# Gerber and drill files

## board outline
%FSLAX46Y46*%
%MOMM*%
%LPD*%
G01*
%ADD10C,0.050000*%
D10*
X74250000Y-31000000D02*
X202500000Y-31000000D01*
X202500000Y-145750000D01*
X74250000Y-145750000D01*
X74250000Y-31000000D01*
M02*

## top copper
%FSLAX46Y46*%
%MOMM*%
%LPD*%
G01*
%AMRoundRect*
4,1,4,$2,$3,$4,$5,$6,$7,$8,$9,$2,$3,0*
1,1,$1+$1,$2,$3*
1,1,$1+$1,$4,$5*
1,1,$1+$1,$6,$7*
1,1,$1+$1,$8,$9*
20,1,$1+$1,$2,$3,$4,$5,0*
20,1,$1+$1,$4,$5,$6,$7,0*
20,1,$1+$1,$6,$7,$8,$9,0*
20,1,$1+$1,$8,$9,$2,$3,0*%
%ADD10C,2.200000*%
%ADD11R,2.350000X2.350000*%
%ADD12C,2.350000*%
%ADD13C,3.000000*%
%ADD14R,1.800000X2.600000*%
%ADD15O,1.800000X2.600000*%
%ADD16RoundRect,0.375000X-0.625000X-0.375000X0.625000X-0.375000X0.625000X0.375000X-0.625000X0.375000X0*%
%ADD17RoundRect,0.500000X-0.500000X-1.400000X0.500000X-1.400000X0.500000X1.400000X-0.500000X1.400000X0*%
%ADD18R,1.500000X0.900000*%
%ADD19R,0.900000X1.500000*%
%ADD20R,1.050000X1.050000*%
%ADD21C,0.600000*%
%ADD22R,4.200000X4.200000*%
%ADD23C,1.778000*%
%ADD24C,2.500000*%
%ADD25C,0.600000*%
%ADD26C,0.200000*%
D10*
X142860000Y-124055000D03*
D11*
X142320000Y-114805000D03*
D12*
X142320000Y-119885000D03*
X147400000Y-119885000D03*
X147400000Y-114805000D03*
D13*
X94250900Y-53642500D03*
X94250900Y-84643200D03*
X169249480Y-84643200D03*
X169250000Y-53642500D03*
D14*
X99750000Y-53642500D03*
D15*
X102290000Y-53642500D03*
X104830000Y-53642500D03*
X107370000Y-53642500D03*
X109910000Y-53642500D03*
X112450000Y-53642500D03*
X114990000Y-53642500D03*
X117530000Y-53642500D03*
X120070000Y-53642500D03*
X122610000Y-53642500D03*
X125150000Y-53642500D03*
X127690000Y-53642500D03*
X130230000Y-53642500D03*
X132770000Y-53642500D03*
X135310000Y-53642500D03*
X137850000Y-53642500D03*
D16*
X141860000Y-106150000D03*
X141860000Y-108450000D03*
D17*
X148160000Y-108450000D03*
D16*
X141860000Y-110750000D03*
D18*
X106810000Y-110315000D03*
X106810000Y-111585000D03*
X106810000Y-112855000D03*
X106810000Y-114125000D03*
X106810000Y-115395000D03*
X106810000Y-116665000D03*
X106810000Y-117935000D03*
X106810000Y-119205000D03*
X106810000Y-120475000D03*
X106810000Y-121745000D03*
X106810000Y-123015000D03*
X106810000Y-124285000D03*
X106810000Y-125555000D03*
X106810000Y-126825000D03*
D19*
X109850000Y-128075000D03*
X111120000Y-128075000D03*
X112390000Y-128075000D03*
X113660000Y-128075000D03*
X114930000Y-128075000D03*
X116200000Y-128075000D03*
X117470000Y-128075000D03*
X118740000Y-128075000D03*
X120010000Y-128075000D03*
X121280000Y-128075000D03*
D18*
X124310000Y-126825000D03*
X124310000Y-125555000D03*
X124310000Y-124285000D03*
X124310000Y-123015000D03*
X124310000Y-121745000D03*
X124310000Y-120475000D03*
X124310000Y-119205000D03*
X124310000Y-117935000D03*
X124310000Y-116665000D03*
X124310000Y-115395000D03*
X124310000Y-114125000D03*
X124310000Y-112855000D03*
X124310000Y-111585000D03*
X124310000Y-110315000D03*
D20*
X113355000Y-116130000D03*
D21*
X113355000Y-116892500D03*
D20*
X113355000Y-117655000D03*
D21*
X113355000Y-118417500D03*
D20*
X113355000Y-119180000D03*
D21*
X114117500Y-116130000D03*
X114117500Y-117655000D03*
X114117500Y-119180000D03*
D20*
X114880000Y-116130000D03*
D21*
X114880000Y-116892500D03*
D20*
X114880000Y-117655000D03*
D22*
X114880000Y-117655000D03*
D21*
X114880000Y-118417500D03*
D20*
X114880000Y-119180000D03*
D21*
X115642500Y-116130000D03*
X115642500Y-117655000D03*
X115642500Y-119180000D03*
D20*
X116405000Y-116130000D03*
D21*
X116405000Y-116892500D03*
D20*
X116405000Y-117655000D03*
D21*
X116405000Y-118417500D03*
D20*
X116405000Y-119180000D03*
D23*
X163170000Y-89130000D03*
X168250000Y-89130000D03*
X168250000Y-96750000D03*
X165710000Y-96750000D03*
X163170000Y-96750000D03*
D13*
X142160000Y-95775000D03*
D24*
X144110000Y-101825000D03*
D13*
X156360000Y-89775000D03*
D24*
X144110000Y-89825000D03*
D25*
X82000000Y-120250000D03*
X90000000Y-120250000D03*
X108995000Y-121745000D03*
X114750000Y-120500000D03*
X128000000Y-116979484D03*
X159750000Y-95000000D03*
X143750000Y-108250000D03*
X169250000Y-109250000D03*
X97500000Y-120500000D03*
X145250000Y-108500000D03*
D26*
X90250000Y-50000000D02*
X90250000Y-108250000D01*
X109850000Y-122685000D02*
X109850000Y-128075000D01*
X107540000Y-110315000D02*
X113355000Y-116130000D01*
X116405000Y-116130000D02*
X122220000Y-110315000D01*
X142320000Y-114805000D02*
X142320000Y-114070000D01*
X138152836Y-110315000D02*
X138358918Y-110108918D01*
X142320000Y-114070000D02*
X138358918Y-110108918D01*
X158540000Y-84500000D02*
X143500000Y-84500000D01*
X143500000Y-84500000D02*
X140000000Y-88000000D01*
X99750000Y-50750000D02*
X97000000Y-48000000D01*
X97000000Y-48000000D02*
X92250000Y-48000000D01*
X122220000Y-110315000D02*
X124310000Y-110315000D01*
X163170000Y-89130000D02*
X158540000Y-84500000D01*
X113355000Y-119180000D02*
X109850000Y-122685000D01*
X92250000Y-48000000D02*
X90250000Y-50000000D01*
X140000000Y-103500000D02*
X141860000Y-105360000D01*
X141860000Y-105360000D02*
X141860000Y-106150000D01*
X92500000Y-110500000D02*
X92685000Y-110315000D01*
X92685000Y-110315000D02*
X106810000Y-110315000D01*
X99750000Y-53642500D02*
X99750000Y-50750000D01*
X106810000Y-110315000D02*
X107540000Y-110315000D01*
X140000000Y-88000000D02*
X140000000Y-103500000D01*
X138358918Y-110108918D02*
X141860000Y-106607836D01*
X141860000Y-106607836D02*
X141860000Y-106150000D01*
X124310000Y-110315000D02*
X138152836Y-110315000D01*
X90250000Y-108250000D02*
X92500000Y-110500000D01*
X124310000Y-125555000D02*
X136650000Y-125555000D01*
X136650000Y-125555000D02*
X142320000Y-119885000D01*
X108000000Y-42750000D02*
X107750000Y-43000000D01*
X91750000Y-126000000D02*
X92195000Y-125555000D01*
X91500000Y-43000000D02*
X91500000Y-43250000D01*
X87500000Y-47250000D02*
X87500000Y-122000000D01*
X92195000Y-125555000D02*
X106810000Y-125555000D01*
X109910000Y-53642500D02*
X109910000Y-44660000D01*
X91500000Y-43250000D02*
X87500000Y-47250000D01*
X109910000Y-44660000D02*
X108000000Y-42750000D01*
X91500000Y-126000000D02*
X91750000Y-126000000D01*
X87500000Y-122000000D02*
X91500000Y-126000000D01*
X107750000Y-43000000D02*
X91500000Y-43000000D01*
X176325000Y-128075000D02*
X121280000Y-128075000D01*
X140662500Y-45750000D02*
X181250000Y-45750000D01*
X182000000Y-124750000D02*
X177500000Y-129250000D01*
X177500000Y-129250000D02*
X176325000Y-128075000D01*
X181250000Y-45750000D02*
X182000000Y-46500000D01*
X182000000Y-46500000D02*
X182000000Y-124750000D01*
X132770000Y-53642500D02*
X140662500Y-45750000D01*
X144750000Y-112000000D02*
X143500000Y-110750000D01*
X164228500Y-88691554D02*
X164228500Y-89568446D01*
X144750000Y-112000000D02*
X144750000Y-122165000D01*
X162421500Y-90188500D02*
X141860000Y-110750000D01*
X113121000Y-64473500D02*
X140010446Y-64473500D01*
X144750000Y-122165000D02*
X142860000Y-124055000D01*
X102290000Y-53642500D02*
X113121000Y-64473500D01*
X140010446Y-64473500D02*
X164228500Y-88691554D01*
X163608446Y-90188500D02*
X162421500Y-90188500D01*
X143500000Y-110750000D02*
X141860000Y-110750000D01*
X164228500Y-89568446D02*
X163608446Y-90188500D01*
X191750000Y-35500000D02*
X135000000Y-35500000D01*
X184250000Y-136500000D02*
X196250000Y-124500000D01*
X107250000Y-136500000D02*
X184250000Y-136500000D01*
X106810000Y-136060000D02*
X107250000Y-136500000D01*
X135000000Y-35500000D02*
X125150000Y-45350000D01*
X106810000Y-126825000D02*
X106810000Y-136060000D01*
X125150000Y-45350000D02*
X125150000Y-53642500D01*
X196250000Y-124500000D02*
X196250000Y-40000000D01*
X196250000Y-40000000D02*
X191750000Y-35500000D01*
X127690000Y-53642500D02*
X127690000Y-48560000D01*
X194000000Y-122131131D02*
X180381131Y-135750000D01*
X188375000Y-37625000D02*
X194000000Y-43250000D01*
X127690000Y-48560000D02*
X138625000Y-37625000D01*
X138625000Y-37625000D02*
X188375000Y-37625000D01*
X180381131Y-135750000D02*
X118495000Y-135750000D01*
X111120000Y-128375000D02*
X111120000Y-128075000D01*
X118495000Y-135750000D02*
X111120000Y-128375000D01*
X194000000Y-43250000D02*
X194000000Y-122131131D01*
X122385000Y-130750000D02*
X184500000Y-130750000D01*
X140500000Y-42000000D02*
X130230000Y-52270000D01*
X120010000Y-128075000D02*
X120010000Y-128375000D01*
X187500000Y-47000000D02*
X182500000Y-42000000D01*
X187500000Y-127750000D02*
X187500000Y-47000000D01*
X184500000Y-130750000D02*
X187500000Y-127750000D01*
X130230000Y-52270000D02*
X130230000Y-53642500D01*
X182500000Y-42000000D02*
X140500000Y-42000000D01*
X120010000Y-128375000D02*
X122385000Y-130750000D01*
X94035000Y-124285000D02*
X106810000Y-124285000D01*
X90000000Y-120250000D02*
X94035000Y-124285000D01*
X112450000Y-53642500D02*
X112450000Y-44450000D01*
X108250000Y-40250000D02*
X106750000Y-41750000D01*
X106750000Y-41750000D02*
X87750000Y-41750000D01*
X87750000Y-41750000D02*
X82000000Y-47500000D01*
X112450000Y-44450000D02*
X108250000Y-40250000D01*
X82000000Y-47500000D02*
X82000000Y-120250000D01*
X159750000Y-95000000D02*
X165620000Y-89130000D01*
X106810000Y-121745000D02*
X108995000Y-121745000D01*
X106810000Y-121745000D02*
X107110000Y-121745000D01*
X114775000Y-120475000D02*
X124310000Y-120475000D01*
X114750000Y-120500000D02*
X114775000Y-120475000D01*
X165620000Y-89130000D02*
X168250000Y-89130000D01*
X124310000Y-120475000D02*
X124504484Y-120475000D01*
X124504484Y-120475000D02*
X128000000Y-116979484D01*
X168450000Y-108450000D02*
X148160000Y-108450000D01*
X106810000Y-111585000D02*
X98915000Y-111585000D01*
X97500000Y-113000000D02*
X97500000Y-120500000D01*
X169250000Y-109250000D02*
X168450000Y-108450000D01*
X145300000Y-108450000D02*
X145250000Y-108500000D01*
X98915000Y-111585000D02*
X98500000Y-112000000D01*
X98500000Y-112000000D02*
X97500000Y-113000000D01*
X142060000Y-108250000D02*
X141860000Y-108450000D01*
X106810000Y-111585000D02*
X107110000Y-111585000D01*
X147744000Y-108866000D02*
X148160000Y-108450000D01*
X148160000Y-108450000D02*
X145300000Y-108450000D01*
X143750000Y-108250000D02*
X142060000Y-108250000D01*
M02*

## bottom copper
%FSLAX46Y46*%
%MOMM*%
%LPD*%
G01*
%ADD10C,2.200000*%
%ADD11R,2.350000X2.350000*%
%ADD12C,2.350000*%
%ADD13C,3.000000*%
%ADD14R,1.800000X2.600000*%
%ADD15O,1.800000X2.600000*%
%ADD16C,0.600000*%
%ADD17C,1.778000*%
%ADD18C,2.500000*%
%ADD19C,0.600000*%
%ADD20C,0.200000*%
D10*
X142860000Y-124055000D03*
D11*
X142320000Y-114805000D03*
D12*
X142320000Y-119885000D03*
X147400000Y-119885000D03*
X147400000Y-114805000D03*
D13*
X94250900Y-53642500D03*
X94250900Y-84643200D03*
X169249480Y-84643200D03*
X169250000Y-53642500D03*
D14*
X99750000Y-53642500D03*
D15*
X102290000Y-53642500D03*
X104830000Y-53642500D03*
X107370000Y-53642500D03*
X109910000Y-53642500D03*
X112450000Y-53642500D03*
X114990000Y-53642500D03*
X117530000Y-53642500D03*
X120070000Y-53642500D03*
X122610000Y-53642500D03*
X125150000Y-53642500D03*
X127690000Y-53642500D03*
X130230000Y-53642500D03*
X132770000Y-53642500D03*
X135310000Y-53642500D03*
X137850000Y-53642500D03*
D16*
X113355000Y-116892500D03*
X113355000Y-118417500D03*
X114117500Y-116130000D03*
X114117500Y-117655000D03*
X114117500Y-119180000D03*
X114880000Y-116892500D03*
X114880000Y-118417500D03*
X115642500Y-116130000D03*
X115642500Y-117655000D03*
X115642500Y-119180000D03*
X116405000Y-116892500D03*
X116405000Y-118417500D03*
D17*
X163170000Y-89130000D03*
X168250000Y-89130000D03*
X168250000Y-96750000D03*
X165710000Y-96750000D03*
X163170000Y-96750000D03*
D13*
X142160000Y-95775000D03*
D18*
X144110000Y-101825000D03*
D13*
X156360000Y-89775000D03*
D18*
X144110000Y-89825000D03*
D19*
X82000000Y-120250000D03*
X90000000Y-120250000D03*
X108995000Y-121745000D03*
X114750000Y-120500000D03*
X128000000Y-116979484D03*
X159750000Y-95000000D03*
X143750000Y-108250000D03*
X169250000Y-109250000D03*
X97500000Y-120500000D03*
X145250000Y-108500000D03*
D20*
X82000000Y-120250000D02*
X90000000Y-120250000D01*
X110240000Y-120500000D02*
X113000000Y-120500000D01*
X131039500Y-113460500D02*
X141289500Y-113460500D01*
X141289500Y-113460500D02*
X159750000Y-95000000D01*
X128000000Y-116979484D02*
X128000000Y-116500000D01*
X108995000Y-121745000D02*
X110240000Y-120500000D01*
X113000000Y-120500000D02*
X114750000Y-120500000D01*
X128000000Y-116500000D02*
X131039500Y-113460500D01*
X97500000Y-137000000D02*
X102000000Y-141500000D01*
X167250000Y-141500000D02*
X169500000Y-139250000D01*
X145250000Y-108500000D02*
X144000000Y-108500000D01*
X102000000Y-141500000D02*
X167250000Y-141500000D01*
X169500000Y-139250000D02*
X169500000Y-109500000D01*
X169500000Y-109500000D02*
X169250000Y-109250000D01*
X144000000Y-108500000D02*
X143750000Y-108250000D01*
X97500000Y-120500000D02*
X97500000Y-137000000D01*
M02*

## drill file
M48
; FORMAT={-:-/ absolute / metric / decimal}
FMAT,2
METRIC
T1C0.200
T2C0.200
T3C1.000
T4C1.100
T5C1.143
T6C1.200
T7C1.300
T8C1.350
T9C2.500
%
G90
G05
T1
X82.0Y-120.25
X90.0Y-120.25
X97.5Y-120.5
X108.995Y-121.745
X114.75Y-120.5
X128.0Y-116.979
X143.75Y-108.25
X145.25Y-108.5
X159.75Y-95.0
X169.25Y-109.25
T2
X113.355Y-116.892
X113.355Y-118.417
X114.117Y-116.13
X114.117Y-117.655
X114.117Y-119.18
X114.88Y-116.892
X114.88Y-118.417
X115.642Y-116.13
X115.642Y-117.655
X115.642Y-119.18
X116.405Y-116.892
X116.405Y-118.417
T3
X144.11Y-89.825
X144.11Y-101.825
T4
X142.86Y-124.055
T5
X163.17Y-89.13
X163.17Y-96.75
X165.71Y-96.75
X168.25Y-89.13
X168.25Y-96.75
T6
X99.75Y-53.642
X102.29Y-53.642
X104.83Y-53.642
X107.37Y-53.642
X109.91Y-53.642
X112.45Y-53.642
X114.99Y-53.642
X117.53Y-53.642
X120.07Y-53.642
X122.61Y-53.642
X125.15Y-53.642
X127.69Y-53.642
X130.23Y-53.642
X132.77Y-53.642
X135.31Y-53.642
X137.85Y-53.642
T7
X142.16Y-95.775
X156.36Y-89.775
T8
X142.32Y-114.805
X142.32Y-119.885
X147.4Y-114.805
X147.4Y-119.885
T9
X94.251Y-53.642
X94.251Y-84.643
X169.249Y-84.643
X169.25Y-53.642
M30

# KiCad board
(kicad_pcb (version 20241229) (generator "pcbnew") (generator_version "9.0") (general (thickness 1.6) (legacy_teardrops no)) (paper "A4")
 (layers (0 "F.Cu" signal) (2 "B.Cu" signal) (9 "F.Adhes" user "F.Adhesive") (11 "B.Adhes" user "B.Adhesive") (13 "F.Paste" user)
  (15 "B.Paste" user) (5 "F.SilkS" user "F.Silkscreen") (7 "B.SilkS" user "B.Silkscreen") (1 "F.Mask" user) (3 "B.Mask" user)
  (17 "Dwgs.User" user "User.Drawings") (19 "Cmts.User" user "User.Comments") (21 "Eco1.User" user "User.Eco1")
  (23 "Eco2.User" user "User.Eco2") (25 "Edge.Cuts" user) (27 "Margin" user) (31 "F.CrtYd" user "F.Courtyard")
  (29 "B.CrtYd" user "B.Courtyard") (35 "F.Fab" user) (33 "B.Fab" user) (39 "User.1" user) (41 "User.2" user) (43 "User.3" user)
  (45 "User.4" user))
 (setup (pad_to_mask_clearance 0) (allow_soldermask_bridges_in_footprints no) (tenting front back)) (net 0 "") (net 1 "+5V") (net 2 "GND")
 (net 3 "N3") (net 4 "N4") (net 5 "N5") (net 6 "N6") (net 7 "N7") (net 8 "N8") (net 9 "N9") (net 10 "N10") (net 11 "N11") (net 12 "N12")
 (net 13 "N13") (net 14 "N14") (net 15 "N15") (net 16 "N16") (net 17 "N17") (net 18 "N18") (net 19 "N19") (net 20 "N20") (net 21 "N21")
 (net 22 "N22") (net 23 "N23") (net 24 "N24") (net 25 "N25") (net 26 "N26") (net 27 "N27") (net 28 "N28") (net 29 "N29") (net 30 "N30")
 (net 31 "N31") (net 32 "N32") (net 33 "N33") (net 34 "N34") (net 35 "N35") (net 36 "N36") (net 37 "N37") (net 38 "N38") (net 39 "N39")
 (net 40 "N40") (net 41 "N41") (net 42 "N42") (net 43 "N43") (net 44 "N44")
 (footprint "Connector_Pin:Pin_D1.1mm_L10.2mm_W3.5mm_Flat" (layer "F.Cu") (at 142.86 124.055)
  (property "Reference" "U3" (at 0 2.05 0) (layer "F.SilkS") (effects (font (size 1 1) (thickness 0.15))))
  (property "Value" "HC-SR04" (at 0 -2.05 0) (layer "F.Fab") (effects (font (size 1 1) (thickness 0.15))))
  (pad "1" thru_hole circle (at 0 0) (size 2.2 2.2) (drill 1.1) (layers "*.Cu" "*.Mask") (remove_unused_layers no) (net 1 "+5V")))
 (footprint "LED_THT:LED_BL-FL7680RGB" (layer "F.Cu") (at 142.32 114.805)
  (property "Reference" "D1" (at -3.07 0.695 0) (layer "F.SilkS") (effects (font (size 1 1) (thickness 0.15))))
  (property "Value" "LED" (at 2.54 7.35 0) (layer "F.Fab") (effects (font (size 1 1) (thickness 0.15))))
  (pad "1" thru_hole rect (at 0 0) (size 2.35 2.35) (drill 1.35) (layers "*.Cu" "*.Mask") (remove_unused_layers no) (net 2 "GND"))
  (pad "2" thru_hole circle (at 0 5.08) (size 2.35 2.35) (drill 1.35) (layers "*.Cu" "*.Mask") (remove_unused_layers no) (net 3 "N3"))
  (pad "3" thru_hole circle (at 5.08 5.08) (size 2.35 2.35) (drill 1.35) (layers "*.Cu" "*.Mask") (remove_unused_layers no))
  (pad "4" thru_hole circle (at 5.08 0) (size 2.35 2.35) (drill 1.35) (layers "*.Cu" "*.Mask") (remove_unused_layers no)))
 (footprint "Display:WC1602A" (layer "F.Cu") (at 99.75 53.6425)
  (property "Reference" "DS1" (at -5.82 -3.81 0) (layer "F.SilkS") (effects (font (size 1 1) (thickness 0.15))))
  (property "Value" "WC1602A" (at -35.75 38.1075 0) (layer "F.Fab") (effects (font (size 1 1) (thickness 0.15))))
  (pad "" thru_hole circle (at -5.4991 0) (size 3 3) (drill 2.5) (layers "*.Cu" "*.Mask") (remove_unused_layers no))
  (pad "" thru_hole circle (at -5.4991 31.0007) (size 3 3) (drill 2.5) (layers "*.Cu" "*.Mask") (remove_unused_layers no))
  (pad "" thru_hole circle (at 69.49948 31.0007) (size 3 3) (drill 2.5) (layers "*.Cu" "*.Mask") (remove_unused_layers no))
  (pad "" thru_hole circle (at 69.5 0) (size 3 3) (drill 2.5) (layers "*.Cu" "*.Mask") (remove_unused_layers no))
  (pad "1" thru_hole rect (at 0 0) (size 1.8 2.6) (drill 1.2) (layers "*.Cu" "*.Mask") (remove_unused_layers no) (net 2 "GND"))
  (pad "2" thru_hole oval (at 2.54 0) (size 1.8 2.6) (drill 1.2) (layers "*.Cu" "*.Mask") (remove_unused_layers no) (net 1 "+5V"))
  (pad "3" thru_hole oval (at 5.08 0) (size 1.8 2.6) (drill 1.2) (layers "*.Cu" "*.Mask") (remove_unused_layers no) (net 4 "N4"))
  (pad "4" thru_hole oval (at 7.62 0) (size 1.8 2.6) (drill 1.2) (layers "*.Cu" "*.Mask") (remove_unused_layers no) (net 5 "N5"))
  (pad "5" thru_hole oval (at 10.16 0) (size 1.8 2.6) (drill 1.2) (layers "*.Cu" "*.Mask") (remove_unused_layers no) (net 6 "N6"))
  (pad "6" thru_hole oval (at 12.7 0) (size 1.8 2.6) (drill 1.2) (layers "*.Cu" "*.Mask") (remove_unused_layers no) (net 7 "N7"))
  (pad "7" thru_hole oval (at 15.24 0) (size 1.8 2.6) (drill 1.2) (layers "*.Cu" "*.Mask") (remove_unused_layers no) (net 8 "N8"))
  (pad "8" thru_hole oval (at 17.78 0) (size 1.8 2.6) (drill 1.2) (layers "*.Cu" "*.Mask") (remove_unused_layers no) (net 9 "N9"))
  (pad "9" thru_hole oval (at 20.32 0) (size 1.8 2.6) (drill 1.2) (layers "*.Cu" "*.Mask") (remove_unused_layers no) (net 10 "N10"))
  (pad "10" thru_hole oval (at 22.86 0) (size 1.8 2.6) (drill 1.2) (layers "*.Cu" "*.Mask") (remove_unused_layers no) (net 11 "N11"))
  (pad "11" thru_hole oval (at 25.4 0) (size 1.8 2.6) (drill 1.2) (layers "*.Cu" "*.Mask") (remove_unused_layers no) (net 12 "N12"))
  (pad "12" thru_hole oval (at 27.94 0) (size 1.8 2.6) (drill 1.2) (layers "*.Cu" "*.Mask") (remove_unused_layers no) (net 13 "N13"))
  (pad "13" thru_hole oval (at 30.48 0) (size 1.8 2.6) (drill 1.2) (layers "*.Cu" "*.Mask") (remove_unused_layers no) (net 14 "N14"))
  (pad "14" thru_hole oval (at 33.02 0) (size 1.8 2.6) (drill 1.2) (layers "*.Cu" "*.Mask") (remove_unused_layers no) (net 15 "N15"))
  (pad "15" thru_hole oval (at 35.56 0) (size 1.8 2.6) (drill 1.2) (layers "*.Cu" "*.Mask") (remove_unused_layers no) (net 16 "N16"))
  (pad "16" thru_hole oval (at 38.1 0) (size 1.8 2.6) (drill 1.2) (layers "*.Cu" "*.Mask") (remove_unused_layers no) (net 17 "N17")))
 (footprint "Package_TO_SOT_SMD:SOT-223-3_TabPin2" (layer "F.Cu") (at 145.01 108.45)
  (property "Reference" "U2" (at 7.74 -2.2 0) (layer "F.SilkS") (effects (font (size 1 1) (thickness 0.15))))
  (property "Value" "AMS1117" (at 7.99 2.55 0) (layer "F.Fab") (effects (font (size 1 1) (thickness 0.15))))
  (pad "1" smd roundrect (at -3.15 -2.3) (size 2 1.5) (layers "F.Cu" "F.Mask" "F.Paste") (roundrect_rratio 0.25) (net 2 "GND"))
  (pad "2" smd roundrect (at -3.15 0) (size 2 1.5) (layers "F.Cu" "F.Mask" "F.Paste") (roundrect_rratio 0.25) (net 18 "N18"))
  (pad "2" smd roundrect (at 3.15 0) (size 2 3.8) (layers "F.Cu" "F.Mask" "F.Paste") (roundrect_rratio 0.25) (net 18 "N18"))
  (pad "3" smd roundrect (at -3.15 2.3) (size 2 1.5) (layers "F.Cu" "F.Mask" "F.Paste") (roundrect_rratio 0.25) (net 1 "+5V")))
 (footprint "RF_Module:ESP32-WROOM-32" (layer "F.Cu") (at 115.56 118.565)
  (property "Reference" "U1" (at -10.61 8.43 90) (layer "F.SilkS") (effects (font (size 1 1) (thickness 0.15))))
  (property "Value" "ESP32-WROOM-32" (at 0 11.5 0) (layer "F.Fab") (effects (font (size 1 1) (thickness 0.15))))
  (pad "1" smd rect (at -8.75 -8.25) (size 1.5 0.9) (layers "F.Cu" "F.Mask" "F.Paste") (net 2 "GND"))
  (pad "2" smd rect (at -8.75 -6.98) (size 1.5 0.9) (layers "F.Cu" "F.Mask" "F.Paste") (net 18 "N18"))
  (pad "3" smd rect (at -8.75 -5.71) (size 1.5 0.9) (layers "F.Cu" "F.Mask" "F.Paste") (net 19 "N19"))
  (pad "4" smd rect (at -8.75 -4.44) (size 1.5 0.9) (layers "F.Cu" "F.Mask" "F.Paste") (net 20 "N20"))
  (pad "5" smd rect (at -8.75 -3.17) (size 1.5 0.9) (layers "F.Cu" "F.Mask" "F.Paste") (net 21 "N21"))
  (pad "6" smd rect (at -8.75 -1.9) (size 1.5 0.9) (layers "F.Cu" "F.Mask" "F.Paste") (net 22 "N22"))
  (pad "7" smd rect (at -8.75 -0.63) (size 1.5 0.9) (layers "F.Cu" "F.Mask" "F.Paste") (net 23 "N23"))
  (pad "8" smd rect (at -8.75 0.64) (size 1.5 0.9) (layers "F.Cu" "F.Mask" "F.Paste") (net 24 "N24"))
  (pad "9" smd rect (at -8.75 1.91) (size 1.5 0.9) (layers "F.Cu" "F.Mask" "F.Paste") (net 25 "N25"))
  (pad "10" smd rect (at -8.75 3.18) (size 1.5 0.9) (layers "F.Cu" "F.Mask" "F.Paste") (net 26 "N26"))
  (pad "11" smd rect (at -8.75 4.45) (size 1.5 0.9) (layers "F.Cu" "F.Mask" "F.Paste") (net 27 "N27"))
  (pad "12" smd rect (at -8.75 5.72) (size 1.5 0.9) (layers "F.Cu" "F.Mask" "F.Paste") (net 7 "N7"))
  (pad "13" smd rect (at -8.75 6.99) (size 1.5 0.9) (layers "F.Cu" "F.Mask" "F.Paste") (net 6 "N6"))
  (pad "14" smd rect (at -8.75 8.26) (size 1.5 0.9) (layers "F.Cu" "F.Mask" "F.Paste") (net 12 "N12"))
  (pad "15" smd rect (at -5.71 9.51 90) (size 1.5 0.9) (layers "F.Cu" "F.Mask" "F.Paste") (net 2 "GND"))
  (pad "16" smd rect (at -4.44 9.51 90) (size 1.5 0.9) (layers "F.Cu" "F.Mask" "F.Paste") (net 13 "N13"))
  (pad "17" smd rect (at -3.17 9.51 90) (size 1.5 0.9) (layers "F.Cu" "F.Mask" "F.Paste") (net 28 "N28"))
  (pad "18" smd rect (at -1.9 9.51 90) (size 1.5 0.9) (layers "F.Cu" "F.Mask" "F.Paste") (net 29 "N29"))
  (pad "19" smd rect (at -0.63 9.51 90) (size 1.5 0.9) (layers "F.Cu" "F.Mask" "F.Paste") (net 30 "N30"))
  (pad "20" smd rect (at 0.64 9.51 90) (size 1.5 0.9) (layers "F.Cu" "F.Mask" "F.Paste") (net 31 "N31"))
  (pad "21" smd rect (at 1.91 9.51 90) (size 1.5 0.9) (layers "F.Cu" "F.Mask" "F.Paste") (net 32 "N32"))
  (pad "22" smd rect (at 3.18 9.51 90) (size 1.5 0.9) (layers "F.Cu" "F.Mask" "F.Paste") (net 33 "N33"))
  (pad "23" smd rect (at 4.45 9.51 90) (size 1.5 0.9) (layers "F.Cu" "F.Mask" "F.Paste") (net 14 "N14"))
  (pad "24" smd rect (at 5.72 9.51 90) (size 1.5 0.9) (layers "F.Cu" "F.Mask" "F.Paste") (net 15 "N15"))
  (pad "25" smd rect (at 8.75 8.26) (size 1.5 0.9) (layers "F.Cu" "F.Mask" "F.Paste") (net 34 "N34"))
  (pad "26" smd rect (at 8.75 6.99) (size 1.5 0.9) (layers "F.Cu" "F.Mask" "F.Paste") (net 3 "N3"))
  (pad "27" smd rect (at 8.75 5.72) (size 1.5 0.9) (layers "F.Cu" "F.Mask" "F.Paste") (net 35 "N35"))
  (pad "28" smd rect (at 8.75 4.45) (size 1.5 0.9) (layers "F.Cu" "F.Mask" "F.Paste") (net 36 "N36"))
  (pad "29" smd rect (at 8.75 3.18) (size 1.5 0.9) (layers "F.Cu" "F.Mask" "F.Paste") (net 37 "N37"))
  (pad "30" smd rect (at 8.75 1.91) (size 1.5 0.9) (layers "F.Cu" "F.Mask" "F.Paste") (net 26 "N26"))
  (pad "31" smd rect (at 8.75 0.64) (size 1.5 0.9) (layers "F.Cu" "F.Mask" "F.Paste") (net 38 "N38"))
  (pad "32" smd rect (at 8.75 -0.63) (size 1.5 0.9) (layers "F.Cu" "F.Mask" "F.Paste") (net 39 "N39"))
  (pad "33" smd rect (at 8.75 -1.9) (size 1.5 0.9) (layers "F.Cu" "F.Mask" "F.Paste") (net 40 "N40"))
  (pad "34" smd rect (at 8.75 -3.17) (size 1.5 0.9) (layers "F.Cu" "F.Mask" "F.Paste") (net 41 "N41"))
  (pad "35" smd rect (at 8.75 -4.44) (size 1.5 0.9) (layers "F.Cu" "F.Mask" "F.Paste") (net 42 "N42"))
  (pad "36" smd rect (at 8.75 -5.71) (size 1.5 0.9) (layers "F.Cu" "F.Mask" "F.Paste") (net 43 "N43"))
  (pad "37" smd rect (at 8.75 -6.98) (size 1.5 0.9) (layers "F.Cu" "F.Mask" "F.Paste") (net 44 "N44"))
  (pad "38" smd rect (at 8.75 -8.25) (size 1.5 0.9) (layers "F.Cu" "F.Mask" "F.Paste") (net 2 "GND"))
  (pad "39" smd rect (at -2.205 -2.435) (size 1.05 1.05) (layers "F.Cu" "F.Paste") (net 2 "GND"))
  (pad "39" thru_hole circle (at -2.205 -1.6725) (size 0.6 0.6) (drill 0.2) (layers "*.Cu" "F.Mask") (remove_unused_layers no) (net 2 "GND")
   (zone_connect 2))
  (pad "39" smd rect (at -2.205 -0.91) (size 1.05 1.05) (layers "F.Cu" "F.Paste") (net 2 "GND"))
  (pad "39" thru_hole circle (at -2.205 -0.1475) (size 0.6 0.6) (drill 0.2) (layers "*.Cu" "F.Mask") (remove_unused_layers no) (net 2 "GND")
   (zone_connect 2))
  (pad "39" smd rect (at -2.205 0.615) (size 1.05 1.05) (layers "F.Cu" "F.Paste") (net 2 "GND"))
  (pad "39" thru_hole circle (at -1.4425 -2.435) (size 0.6 0.6) (drill 0.2) (layers "*.Cu" "F.Mask") (remove_unused_layers no) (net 2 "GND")
   (zone_connect 2))
  (pad "39" thru_hole circle (at -1.4425 -0.91) (size 0.6 0.6) (drill 0.2) (layers "*.Cu" "F.Mask") (remove_unused_layers no) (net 2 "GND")
   (zone_connect 2))
  (pad "39" thru_hole circle (at -1.4425 0.615) (size 0.6 0.6) (drill 0.2) (layers "*.Cu" "F.Mask") (remove_unused_layers no) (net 2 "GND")
   (zone_connect 2))
  (pad "39" smd rect (at -0.68 -2.435) (size 1.05 1.05) (layers "F.Cu" "F.Paste") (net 2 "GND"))
  (pad "39" thru_hole circle (at -0.68 -1.6725) (size 0.6 0.6) (drill 0.2) (layers "*.Cu" "F.Mask") (remove_unused_layers no) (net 2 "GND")
   (zone_connect 2))
  (pad "39" smd rect (at -0.68 -0.91) (size 1.05 1.05) (layers "F.Cu" "F.Paste") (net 2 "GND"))
  (pad "39" smd rect (at -0.68 -0.91) (size 4.2 4.2) (layers "F.Cu" "F.Mask") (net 2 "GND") (zone_connect 2))
  (pad "39" thru_hole circle (at -0.68 -0.1475) (size 0.6 0.6) (drill 0.2) (layers "*.Cu" "F.Mask") (remove_unused_layers no) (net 2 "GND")
   (zone_connect 2))
  (pad "39" smd rect (at -0.68 0.615) (size 1.05 1.05) (layers "F.Cu" "F.Paste") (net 2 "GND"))
  (pad "39" thru_hole circle (at 0.0825 -2.435) (size 0.6 0.6) (drill 0.2) (layers "*.Cu" "F.Mask") (remove_unused_layers no) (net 2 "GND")
   (zone_connect 2))
  (pad "39" thru_hole circle (at 0.0825 -0.91) (size 0.6 0.6) (drill 0.2) (layers "*.Cu" "F.Mask") (remove_unused_layers no) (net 2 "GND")
   (zone_connect 2))
  (pad "39" thru_hole circle (at 0.0825 0.615) (size 0.6 0.6) (drill 0.2) (layers "*.Cu" "F.Mask") (remove_unused_layers no) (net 2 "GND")
   (zone_connect 2))
  (pad "39" smd rect (at 0.845 -2.435) (size 1.05 1.05) (layers "F.Cu" "F.Paste") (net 2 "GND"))
  (pad "39" thru_hole circle (at 0.845 -1.6725) (size 0.6 0.6) (drill 0.2) (layers "*.Cu" "F.Mask") (remove_unused_layers no) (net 2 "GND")
   (zone_connect 2))
  (pad "39" smd rect (at 0.845 -0.91) (size 1.05 1.05) (layers "F.Cu" "F.Paste") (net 2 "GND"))
  (pad "39" thru_hole circle (at 0.845 -0.1475) (size 0.6 0.6) (drill 0.2) (layers "*.Cu" "F.Mask") (remove_unused_layers no) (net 2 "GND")
   (zone_connect 2))
  (pad "39" smd rect (at 0.845 0.615) (size 1.05 1.05) (layers "F.Cu" "F.Paste") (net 2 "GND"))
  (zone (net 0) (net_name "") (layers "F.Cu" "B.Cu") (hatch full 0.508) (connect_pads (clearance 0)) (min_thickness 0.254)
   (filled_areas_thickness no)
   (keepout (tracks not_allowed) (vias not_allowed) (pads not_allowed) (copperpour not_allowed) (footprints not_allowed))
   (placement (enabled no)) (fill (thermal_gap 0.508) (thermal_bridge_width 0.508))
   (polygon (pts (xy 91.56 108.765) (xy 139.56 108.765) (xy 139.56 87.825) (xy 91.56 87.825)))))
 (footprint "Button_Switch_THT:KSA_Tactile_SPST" (layer "F.Cu") (at 163.17 89.13)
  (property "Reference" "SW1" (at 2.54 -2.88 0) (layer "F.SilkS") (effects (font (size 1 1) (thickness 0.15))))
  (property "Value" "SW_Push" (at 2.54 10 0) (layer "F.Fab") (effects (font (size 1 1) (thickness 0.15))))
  (pad "1" thru_hole circle (at 0 0) (size 1.778 1.778) (drill 1.143) (layers "*.Cu" "*.Mask") (remove_unused_layers no) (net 2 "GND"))
  (pad "2" thru_hole circle (at 5.08 0) (size 1.778 1.778) (drill 1.143) (layers "*.Cu" "*.Mask") (remove_unused_layers no) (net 26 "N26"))
  (pad "3" thru_hole circle (at 5.08 7.62) (size 1.778 1.778) (drill 1.143) (layers "*.Cu" "*.Mask") (remove_unused_layers no))
  (pad "4" thru_hole circle (at 2.54 7.62) (size 1.778 1.778) (drill 1.143) (layers "*.Cu" "*.Mask") (remove_unused_layers no))
  (pad "5" thru_hole circle (at 0 7.62) (size 1.778 1.778) (drill 1.143) (layers "*.Cu" "*.Mask") (remove_unused_layers no)))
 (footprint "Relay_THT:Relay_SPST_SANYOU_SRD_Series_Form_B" (layer "F.Cu") (at 142.16 95.775)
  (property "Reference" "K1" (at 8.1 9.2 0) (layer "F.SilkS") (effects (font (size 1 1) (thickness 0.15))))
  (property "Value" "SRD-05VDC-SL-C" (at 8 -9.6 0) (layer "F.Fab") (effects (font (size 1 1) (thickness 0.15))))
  (pad "1" thru_hole circle (at 0 0 90) (size 3 3) (drill 1.3) (layers "*.Cu" "*.Mask") (remove_unused_layers no))
  (pad "2" thru_hole circle (at 1.95 6.05 90) (size 2.5 2.5) (drill 1) (layers "*.Cu" "*.Mask") (remove_unused_layers no))
  (pad "4" thru_hole circle (at 14.2 -6 90) (size 3 3) (drill 1.3) (layers "*.Cu" "*.Mask") (remove_unused_layers no))
  (pad "5" thru_hole circle (at 1.95 -5.95 90) (size 2.5 2.5) (drill 1) (layers "*.Cu" "*.Mask") (remove_unused_layers no)))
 (gr_rect (start 74.25 31) (end 202.5 145.75) (stroke (width 0.05) (type default)) (fill no) (layer "Edge.Cuts"))
 (segment (start 90.25 50) (end 90.25 108.25) (width 0.2) (layer "F.Cu") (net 2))
 (segment (start 109.85 122.685) (end 109.85 128.075) (width 0.2) (layer "F.Cu") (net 2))
 (segment (start 107.54 110.315) (end 113.355 116.13) (width 0.2) (layer "F.Cu") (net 2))
 (segment (start 116.405 116.13) (end 122.22 110.315) (width 0.2) (layer "F.Cu") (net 2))
 (segment (start 142.32 114.805) (end 142.32 114.07) (width 0.2) (layer "F.Cu") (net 2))
 (segment (start 138.152836 110.315) (end 138.358918 110.108918) (width 0.2) (layer "F.Cu") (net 2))
 (segment (start 142.32 114.07) (end 138.358918 110.108918) (width 0.2) (layer "F.Cu") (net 2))
 (segment (start 158.54 84.5) (end 143.5 84.5) (width 0.2) (layer "F.Cu") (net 2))
 (segment (start 143.5 84.5) (end 140 88) (width 0.2) (layer "F.Cu") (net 2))
 (segment (start 99.75 50.75) (end 97 48) (width 0.2) (layer "F.Cu") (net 2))
 (segment (start 97 48) (end 92.25 48) (width 0.2) (layer "F.Cu") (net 2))
 (segment (start 122.22 110.315) (end 124.31 110.315) (width 0.2) (layer "F.Cu") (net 2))
 (segment (start 163.17 89.13) (end 158.54 84.5) (width 0.2) (layer "F.Cu") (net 2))
 (segment (start 113.355 119.18) (end 109.85 122.685) (width 0.2) (layer "F.Cu") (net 2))
 (segment (start 92.25 48) (end 90.25 50) (width 0.2) (layer "F.Cu") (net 2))
 (segment (start 140 103.5) (end 141.86 105.36) (width 0.2) (layer "F.Cu") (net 2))
 (segment (start 141.86 105.36) (end 141.86 106.15) (width 0.2) (layer "F.Cu") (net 2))
 (segment (start 92.5 110.5) (end 92.685 110.315) (width 0.2) (layer "F.Cu") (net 2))
 (segment (start 92.685 110.315) (end 106.81 110.315) (width 0.2) (layer "F.Cu") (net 2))
 (segment (start 99.75 53.6425) (end 99.75 50.75) (width 0.2) (layer "F.Cu") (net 2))
 (segment (start 106.81 110.315) (end 107.54 110.315) (width 0.2) (layer "F.Cu") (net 2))
 (segment (start 140 88) (end 140 103.5) (width 0.2) (layer "F.Cu") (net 2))
 (segment (start 138.358918 110.108918) (end 141.86 106.607836) (width 0.2) (layer "F.Cu") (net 2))
 (segment (start 141.86 106.607836) (end 141.86 106.15) (width 0.2) (layer "F.Cu") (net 2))
 (segment (start 124.31 110.315) (end 138.152836 110.315) (width 0.2) (layer "F.Cu") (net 2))
 (segment (start 90.25 108.25) (end 92.5 110.5) (width 0.2) (layer "F.Cu") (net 2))
 (segment (start 124.31 125.555) (end 136.65 125.555) (width 0.2) (layer "F.Cu") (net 3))
 (segment (start 136.65 125.555) (end 142.32 119.885) (width 0.2) (layer "F.Cu") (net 3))
 (segment (start 108 42.75) (end 107.75 43) (width 0.2) (layer "F.Cu") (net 6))
 (segment (start 91.75 126) (end 92.195 125.555) (width 0.2) (layer "F.Cu") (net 6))
 (segment (start 91.5 43) (end 91.5 43.25) (width 0.2) (layer "F.Cu") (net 6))
 (segment (start 87.5 47.25) (end 87.5 122) (width 0.2) (layer "F.Cu") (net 6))
 (segment (start 92.195 125.555) (end 106.81 125.555) (width 0.2) (layer "F.Cu") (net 6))
 (segment (start 109.91 53.6425) (end 109.91 44.66) (width 0.2) (layer "F.Cu") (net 6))
 (segment (start 91.5 43.25) (end 87.5 47.25) (width 0.2) (layer "F.Cu") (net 6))
 (segment (start 109.91 44.66) (end 108 42.75) (width 0.2) (layer "F.Cu") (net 6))
 (segment (start 91.5 126) (end 91.75 126) (width 0.2) (layer "F.Cu") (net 6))
 (segment (start 87.5 122) (end 91.5 126) (width 0.2) (layer "F.Cu") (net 6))
 (segment (start 107.75 43) (end 91.5 43) (width 0.2) (layer "F.Cu") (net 6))
 (segment (start 176.325 128.075) (end 121.28 128.075) (width 0.2) (layer "F.Cu") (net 15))
 (segment (start 140.6625 45.75) (end 181.25 45.75) (width 0.2) (layer "F.Cu") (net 15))
 (segment (start 182 124.75) (end 177.5 129.25) (width 0.2) (layer "F.Cu") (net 15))
 (segment (start 177.5 129.25) (end 176.325 128.075) (width 0.2) (layer "F.Cu") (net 15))
 (segment (start 181.25 45.75) (end 182 46.5) (width 0.2) (layer "F.Cu") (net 15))
 (segment (start 182 46.5) (end 182 124.75) (width 0.2) (layer "F.Cu") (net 15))
 (segment (start 132.77 53.6425) (end 140.6625 45.75) (width 0.2) (layer "F.Cu") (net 15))
 (segment (start 144.75 112) (end 143.5 110.75) (width 0.2) (layer "F.Cu") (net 1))
 (segment (start 164.2285 88.691554) (end 164.2285 89.568446) (width 0.2) (layer "F.Cu") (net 1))
 (segment (start 144.75 112) (end 144.75 122.165) (width 0.2) (layer "F.Cu") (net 1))
 (segment (start 162.4215 90.1885) (end 141.86 110.75) (width 0.2) (layer "F.Cu") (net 1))
 (segment (start 113.121 64.4735) (end 140.010446 64.4735) (width 0.2) (layer "F.Cu") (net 1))
 (segment (start 144.75 122.165) (end 142.86 124.055) (width 0.2) (layer "F.Cu") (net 1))
 (segment (start 102.29 53.6425) (end 113.121 64.4735) (width 0.2) (layer "F.Cu") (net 1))
 (segment (start 140.010446 64.4735) (end 164.2285 88.691554) (width 0.2) (layer "F.Cu") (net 1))
 (segment (start 163.608446 90.1885) (end 162.4215 90.1885) (width 0.2) (layer "F.Cu") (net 1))
 (segment (start 143.5 110.75) (end 141.86 110.75) (width 0.2) (layer "F.Cu") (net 1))
 (segment (start 164.2285 89.568446) (end 163.608446 90.1885) (width 0.2) (layer "F.Cu") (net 1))
 (segment (start 191.75 35.5) (end 135 35.5) (width 0.2) (layer "F.Cu") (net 12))
 (segment (start 184.25 136.5) (end 196.25 124.5) (width 0.2) (layer "F.Cu") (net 12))
 (segment (start 107.25 136.5) (end 184.25 136.5) (width 0.2) (layer "F.Cu") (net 12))
 (segment (start 106.81 136.06) (end 107.25 136.5) (width 0.2) (layer "F.Cu") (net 12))
 (segment (start 135 35.5) (end 125.15 45.35) (width 0.2) (layer "F.Cu") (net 12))
 (segment (start 106.81 126.825) (end 106.81 136.06) (width 0.2) (layer "F.Cu") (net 12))
 (segment (start 125.15 45.35) (end 125.15 53.6425) (width 0.2) (layer "F.Cu") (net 12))
 (segment (start 196.25 124.5) (end 196.25 40) (width 0.2) (layer "F.Cu") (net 12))
 (segment (start 196.25 40) (end 191.75 35.5) (width 0.2) (layer "F.Cu") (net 12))
 (segment (start 127.69 53.6425) (end 127.69 48.56) (width 0.2) (layer "F.Cu") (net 13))
 (segment (start 194 122.131131) (end 180.381131 135.75) (width 0.2) (layer "F.Cu") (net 13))
 (segment (start 188.375 37.625) (end 194 43.25) (width 0.2) (layer "F.Cu") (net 13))
 (segment (start 127.69 48.56) (end 138.625 37.625) (width 0.2) (layer "F.Cu") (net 13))
 (segment (start 138.625 37.625) (end 188.375 37.625) (width 0.2) (layer "F.Cu") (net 13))
 (segment (start 180.381131 135.75) (end 118.495 135.75) (width 0.2) (layer "F.Cu") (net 13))
 (segment (start 111.12 128.375) (end 111.12 128.075) (width 0.2) (layer "F.Cu") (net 13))
 (segment (start 118.495 135.75) (end 111.12 128.375) (width 0.2) (layer "F.Cu") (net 13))
 (segment (start 194 43.25) (end 194 122.131131) (width 0.2) (layer "F.Cu") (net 13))
 (segment (start 122.385 130.75) (end 184.5 130.75) (width 0.2) (layer "F.Cu") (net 14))
 (segment (start 140.5 42) (end 130.23 52.27) (width 0.2) (layer "F.Cu") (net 14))
 (segment (start 120.01 128.075) (end 120.01 128.375) (width 0.2) (layer "F.Cu") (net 14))
 (segment (start 187.5 47) (end 182.5 42) (width 0.2) (layer "F.Cu") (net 14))
 (segment (start 187.5 127.75) (end 187.5 47) (width 0.2) (layer "F.Cu") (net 14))
 (segment (start 184.5 130.75) (end 187.5 127.75) (width 0.2) (layer "F.Cu") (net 14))
 (segment (start 130.23 52.27) (end 130.23 53.6425) (width 0.2) (layer "F.Cu") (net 14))
 (segment (start 182.5 42) (end 140.5 42) (width 0.2) (layer "F.Cu") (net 14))
 (segment (start 120.01 128.375) (end 122.385 130.75) (width 0.2) (layer "F.Cu") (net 14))
 (segment (start 94.035 124.285) (end 106.81 124.285) (width 0.2) (layer "F.Cu") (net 7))
 (segment (start 90 120.25) (end 94.035 124.285) (width 0.2) (layer "F.Cu") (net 7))
 (segment (start 112.45 53.6425) (end 112.45 44.45) (width 0.2) (layer "F.Cu") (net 7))
 (segment (start 108.25 40.25) (end 106.75 41.75) (width 0.2) (layer "F.Cu") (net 7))
 (segment (start 106.75 41.75) (end 87.75 41.75) (width 0.2) (layer "F.Cu") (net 7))
 (segment (start 87.75 41.75) (end 82 47.5) (width 0.2) (layer "F.Cu") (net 7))
 (segment (start 112.45 44.45) (end 108.25 40.25) (width 0.2) (layer "F.Cu") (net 7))
 (segment (start 82 47.5) (end 82 120.25) (width 0.2) (layer "F.Cu") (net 7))
 (via (at 82 120.25) (size 0.6) (drill 0.2) (layers "F.Cu" "B.Cu") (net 7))
 (via (at 90 120.25) (size 0.6) (drill 0.2) (layers "F.Cu" "B.Cu") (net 7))
 (segment (start 82 120.25) (end 90 120.25) (width 0.2) (layer "B.Cu") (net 7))
 (segment (start 159.75 95) (end 165.62 89.13) (width 0.2) (layer "F.Cu") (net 26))
 (segment (start 106.81 121.745) (end 108.995 121.745) (width 0.2) (layer "F.Cu") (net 26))
 (segment (start 106.81 121.745) (end 107.11 121.745) (width 0.2) (layer "F.Cu") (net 26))
 (segment (start 114.775 120.475) (end 124.31 120.475) (width 0.2) (layer "F.Cu") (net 26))
 (segment (start 114.75 120.5) (end 114.775 120.475) (width 0.2) (layer "F.Cu") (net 26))
 (segment (start 165.62 89.13) (end 168.25 89.13) (width 0.2) (layer "F.Cu") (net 26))
 (segment (start 124.31 120.475) (end 124.504484 120.475) (width 0.2) (layer "F.Cu") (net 26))
 (segment (start 124.504484 120.475) (end 128 116.979484) (width 0.2) (layer "F.Cu") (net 26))
 (via (at 108.995 121.745) (size 0.6) (drill 0.2) (layers "F.Cu" "B.Cu") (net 26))
 (via (at 114.75 120.5) (size 0.6) (drill 0.2) (layers "F.Cu" "B.Cu") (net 26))
 (via (at 128 116.979484) (size 0.6) (drill 0.2) (layers "F.Cu" "B.Cu") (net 26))
 (via (at 159.75 95) (size 0.6) (drill 0.2) (layers "F.Cu" "B.Cu") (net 26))
 (segment (start 110.24 120.5) (end 113 120.5) (width 0.2) (layer "B.Cu") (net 26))
 (segment (start 131.0395 113.4605) (end 141.2895 113.4605) (width 0.2) (layer "B.Cu") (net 26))
 (segment (start 141.2895 113.4605) (end 159.75 95) (width 0.2) (layer "B.Cu") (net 26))
 (segment (start 128 116.979484) (end 128 116.5) (width 0.2) (layer "B.Cu") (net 26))
 (segment (start 108.995 121.745) (end 110.24 120.5) (width 0.2) (layer "B.Cu") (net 26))
 (segment (start 113 120.5) (end 114.75 120.5) (width 0.2) (layer "B.Cu") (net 26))
 (segment (start 128 116.5) (end 131.0395 113.4605) (width 0.2) (layer "B.Cu") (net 26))
 (segment (start 168.45 108.45) (end 148.16 108.45) (width 0.2) (layer "F.Cu") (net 18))
 (segment (start 106.81 111.585) (end 98.915 111.585) (width 0.2) (layer "F.Cu") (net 18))
 (segment (start 97.5 113) (end 97.5 120.5) (width 0.2) (layer "F.Cu") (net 18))
 (segment (start 169.25 109.25) (end 168.45 108.45) (width 0.2) (layer "F.Cu") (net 18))
 (segment (start 145.3 108.45) (end 145.25 108.5) (width 0.2) (layer "F.Cu") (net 18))
 (segment (start 98.915 111.585) (end 98.5 112) (width 0.2) (layer "F.Cu") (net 18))
 (segment (start 98.5 112) (end 97.5 113) (width 0.2) (layer "F.Cu") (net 18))
 (segment (start 142.06 108.25) (end 141.86 108.45) (width 0.2) (layer "F.Cu") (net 18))
 (segment (start 106.81 111.585) (end 107.11 111.585) (width 0.2) (layer "F.Cu") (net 18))
 (segment (start 147.744 108.866) (end 148.16 108.45) (width 0.2) (layer "F.Cu") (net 18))
 (segment (start 148.16 108.45) (end 145.3 108.45) (width 0.2) (layer "F.Cu") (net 18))
 (segment (start 143.75 108.25) (end 142.06 108.25) (width 0.2) (layer "F.Cu") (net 18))
 (via (at 143.75 108.25) (size 0.6) (drill 0.2) (layers "F.Cu" "B.Cu") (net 18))
 (via (at 169.25 109.25) (size 0.6) (drill 0.2) (layers "F.Cu" "B.Cu") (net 18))
 (via (at 97.5 120.5) (size 0.6) (drill 0.2) (layers "F.Cu" "B.Cu") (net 18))
 (via (at 145.25 108.5) (size 0.6) (drill 0.2) (layers "F.Cu" "B.Cu") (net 18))
 (segment (start 97.5 137) (end 102 141.5) (width 0.2) (layer "B.Cu") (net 18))
 (segment (start 167.25 141.5) (end 169.5 139.25) (width 0.2) (layer "B.Cu") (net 18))
 (segment (start 145.25 108.5) (end 144 108.5) (width 0.2) (layer "B.Cu") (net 18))
 (segment (start 102 141.5) (end 167.25 141.5) (width 0.2) (layer "B.Cu") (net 18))
 (segment (start 169.5 139.25) (end 169.5 109.5) (width 0.2) (layer "B.Cu") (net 18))
 (segment (start 169.5 109.5) (end 169.25 109.25) (width 0.2) (layer "B.Cu") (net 18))
 (segment (start 144 108.5) (end 143.75 108.25) (width 0.2) (layer "B.Cu") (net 18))
 (segment (start 97.5 120.5) (end 97.5 137) (width 0.2) (layer "B.Cu") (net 18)))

